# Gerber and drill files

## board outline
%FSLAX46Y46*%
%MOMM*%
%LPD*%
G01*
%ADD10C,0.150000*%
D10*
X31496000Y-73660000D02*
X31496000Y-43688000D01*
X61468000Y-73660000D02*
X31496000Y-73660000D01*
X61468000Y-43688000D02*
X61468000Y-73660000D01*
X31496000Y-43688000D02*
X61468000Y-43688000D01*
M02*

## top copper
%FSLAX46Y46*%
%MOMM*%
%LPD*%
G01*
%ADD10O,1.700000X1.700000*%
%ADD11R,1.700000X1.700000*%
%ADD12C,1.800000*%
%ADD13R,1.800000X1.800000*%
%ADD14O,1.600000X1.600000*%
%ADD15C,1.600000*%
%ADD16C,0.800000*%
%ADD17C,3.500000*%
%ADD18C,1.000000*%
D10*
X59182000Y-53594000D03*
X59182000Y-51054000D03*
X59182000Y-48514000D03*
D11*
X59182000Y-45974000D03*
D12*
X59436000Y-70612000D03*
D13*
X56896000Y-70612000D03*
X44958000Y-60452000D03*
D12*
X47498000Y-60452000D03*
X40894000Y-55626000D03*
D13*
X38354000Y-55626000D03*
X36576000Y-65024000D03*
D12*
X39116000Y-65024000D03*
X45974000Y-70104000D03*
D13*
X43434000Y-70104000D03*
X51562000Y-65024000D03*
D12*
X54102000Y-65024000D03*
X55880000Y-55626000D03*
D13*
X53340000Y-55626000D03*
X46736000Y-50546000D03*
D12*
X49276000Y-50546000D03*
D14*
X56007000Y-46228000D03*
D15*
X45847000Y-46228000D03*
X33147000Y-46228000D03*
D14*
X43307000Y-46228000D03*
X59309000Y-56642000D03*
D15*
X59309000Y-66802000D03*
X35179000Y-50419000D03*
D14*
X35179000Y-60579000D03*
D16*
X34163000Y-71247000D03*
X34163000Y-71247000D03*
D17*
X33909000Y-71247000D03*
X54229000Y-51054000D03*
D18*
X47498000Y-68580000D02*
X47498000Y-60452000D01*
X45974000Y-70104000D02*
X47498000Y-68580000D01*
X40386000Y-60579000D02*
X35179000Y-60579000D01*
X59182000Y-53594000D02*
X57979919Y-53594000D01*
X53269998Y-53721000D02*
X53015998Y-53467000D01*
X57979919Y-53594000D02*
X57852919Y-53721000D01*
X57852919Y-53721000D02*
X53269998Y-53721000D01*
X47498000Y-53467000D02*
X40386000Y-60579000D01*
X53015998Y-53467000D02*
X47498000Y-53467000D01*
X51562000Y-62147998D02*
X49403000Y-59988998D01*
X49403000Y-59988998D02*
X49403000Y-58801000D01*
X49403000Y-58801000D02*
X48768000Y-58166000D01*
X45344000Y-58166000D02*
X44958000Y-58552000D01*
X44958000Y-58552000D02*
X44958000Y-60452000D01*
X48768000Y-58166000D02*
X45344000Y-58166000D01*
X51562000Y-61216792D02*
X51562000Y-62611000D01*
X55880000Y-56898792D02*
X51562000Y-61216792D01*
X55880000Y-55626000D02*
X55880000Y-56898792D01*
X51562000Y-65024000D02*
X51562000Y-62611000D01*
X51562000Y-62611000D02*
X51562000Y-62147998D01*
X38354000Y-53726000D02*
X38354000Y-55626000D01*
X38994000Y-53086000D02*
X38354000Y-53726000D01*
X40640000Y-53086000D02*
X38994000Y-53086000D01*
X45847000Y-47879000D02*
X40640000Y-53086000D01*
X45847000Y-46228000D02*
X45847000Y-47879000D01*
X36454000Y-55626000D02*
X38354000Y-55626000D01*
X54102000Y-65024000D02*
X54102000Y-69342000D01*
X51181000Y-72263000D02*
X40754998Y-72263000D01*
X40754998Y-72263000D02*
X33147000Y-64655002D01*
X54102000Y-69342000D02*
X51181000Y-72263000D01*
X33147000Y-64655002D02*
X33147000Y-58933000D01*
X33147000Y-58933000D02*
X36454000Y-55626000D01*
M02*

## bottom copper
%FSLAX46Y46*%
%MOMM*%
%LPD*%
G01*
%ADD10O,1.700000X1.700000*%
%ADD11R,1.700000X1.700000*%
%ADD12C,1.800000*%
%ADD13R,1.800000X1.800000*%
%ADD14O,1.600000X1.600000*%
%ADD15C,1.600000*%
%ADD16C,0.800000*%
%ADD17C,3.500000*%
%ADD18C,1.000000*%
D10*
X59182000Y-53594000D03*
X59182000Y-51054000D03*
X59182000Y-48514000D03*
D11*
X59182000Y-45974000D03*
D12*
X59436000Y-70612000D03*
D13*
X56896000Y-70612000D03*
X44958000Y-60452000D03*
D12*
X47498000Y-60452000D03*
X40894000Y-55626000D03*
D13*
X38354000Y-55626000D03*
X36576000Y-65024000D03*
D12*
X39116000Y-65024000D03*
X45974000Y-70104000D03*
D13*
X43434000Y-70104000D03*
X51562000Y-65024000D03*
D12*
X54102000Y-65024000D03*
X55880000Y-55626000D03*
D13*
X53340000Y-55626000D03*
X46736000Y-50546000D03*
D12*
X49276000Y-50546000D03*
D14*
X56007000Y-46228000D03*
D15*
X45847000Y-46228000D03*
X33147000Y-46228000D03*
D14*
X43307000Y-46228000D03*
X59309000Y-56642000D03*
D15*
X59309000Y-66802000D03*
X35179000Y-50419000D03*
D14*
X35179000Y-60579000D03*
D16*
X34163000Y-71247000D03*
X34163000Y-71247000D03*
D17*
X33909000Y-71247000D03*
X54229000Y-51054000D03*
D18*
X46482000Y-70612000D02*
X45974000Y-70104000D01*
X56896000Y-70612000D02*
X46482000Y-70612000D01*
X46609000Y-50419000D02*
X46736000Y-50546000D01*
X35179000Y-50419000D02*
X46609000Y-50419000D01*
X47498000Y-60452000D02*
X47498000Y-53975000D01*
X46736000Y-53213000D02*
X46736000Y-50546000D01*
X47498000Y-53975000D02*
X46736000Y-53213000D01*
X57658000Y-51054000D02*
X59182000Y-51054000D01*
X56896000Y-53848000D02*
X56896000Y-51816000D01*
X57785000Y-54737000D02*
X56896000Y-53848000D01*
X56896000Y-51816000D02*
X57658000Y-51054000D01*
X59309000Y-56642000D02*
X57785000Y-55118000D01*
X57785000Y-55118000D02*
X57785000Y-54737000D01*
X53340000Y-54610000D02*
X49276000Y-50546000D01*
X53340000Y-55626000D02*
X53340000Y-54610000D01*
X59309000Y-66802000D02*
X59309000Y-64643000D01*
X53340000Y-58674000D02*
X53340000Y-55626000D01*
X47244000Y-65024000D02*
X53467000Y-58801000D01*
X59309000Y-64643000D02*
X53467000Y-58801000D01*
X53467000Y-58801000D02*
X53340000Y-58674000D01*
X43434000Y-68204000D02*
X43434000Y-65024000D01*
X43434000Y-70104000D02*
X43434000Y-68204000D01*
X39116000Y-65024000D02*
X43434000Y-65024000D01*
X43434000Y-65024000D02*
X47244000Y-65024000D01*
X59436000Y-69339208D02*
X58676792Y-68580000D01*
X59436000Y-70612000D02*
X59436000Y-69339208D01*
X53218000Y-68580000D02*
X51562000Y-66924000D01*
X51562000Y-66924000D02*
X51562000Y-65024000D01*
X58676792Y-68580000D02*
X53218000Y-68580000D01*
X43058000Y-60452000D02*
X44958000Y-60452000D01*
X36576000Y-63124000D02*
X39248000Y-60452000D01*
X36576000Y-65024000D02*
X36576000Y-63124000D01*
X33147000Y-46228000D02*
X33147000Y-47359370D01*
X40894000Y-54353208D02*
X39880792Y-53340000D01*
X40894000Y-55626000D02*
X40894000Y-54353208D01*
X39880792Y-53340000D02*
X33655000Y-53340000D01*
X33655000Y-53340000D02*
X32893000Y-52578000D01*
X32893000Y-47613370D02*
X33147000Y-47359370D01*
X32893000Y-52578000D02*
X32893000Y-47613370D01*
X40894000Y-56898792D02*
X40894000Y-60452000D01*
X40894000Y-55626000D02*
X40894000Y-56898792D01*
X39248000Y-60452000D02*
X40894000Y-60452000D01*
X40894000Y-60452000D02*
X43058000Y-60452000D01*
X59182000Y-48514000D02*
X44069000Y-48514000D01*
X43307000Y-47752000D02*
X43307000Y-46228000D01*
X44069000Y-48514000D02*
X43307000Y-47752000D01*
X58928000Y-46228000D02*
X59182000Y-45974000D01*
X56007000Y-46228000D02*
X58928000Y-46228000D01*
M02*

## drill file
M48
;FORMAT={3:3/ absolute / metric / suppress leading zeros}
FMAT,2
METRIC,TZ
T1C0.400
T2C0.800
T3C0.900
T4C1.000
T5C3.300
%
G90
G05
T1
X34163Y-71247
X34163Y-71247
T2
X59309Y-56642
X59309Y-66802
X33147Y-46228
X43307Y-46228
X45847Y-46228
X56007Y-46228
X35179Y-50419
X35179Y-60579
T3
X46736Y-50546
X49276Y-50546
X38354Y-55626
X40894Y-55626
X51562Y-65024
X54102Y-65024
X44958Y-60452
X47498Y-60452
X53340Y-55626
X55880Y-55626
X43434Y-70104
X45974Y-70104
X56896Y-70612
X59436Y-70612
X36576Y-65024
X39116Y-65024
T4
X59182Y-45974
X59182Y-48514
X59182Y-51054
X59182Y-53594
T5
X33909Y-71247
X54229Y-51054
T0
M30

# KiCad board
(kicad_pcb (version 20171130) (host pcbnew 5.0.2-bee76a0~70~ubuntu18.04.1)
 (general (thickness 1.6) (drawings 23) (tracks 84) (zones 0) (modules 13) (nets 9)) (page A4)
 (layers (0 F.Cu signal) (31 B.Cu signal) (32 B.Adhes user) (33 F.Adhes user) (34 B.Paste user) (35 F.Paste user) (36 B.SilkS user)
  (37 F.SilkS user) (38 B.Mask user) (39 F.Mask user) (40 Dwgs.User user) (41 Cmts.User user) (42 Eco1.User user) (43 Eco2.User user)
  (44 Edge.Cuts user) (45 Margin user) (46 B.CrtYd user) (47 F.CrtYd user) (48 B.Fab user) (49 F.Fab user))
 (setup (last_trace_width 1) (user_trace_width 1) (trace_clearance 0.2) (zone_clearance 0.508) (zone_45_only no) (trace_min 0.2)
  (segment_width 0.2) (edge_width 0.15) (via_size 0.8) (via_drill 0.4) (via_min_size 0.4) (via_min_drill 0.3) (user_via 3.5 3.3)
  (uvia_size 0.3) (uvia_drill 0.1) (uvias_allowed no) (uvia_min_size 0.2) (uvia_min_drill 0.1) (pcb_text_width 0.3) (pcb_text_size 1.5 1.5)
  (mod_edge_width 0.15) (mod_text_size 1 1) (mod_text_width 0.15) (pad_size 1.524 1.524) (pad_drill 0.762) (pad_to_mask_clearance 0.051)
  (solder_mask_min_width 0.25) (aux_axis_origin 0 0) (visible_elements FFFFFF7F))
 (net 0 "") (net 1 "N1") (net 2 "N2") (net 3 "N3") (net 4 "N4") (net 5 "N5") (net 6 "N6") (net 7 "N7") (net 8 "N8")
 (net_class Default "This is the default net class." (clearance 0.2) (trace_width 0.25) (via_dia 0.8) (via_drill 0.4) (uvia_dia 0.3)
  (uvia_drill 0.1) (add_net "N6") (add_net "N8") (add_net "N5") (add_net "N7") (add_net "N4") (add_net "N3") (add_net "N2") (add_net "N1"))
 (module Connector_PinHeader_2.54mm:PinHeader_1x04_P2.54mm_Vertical (layer F.Cu) (at 59.182 45.974)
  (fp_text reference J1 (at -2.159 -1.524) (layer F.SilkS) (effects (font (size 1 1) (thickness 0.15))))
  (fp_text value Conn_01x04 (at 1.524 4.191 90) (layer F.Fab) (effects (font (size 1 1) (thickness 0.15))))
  (pad 4 thru_hole oval (at 0 7.62) (size 1.7 1.7) (drill 1) (layers *.Cu *.Mask) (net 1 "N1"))
  (pad 3 thru_hole oval (at 0 5.08) (size 1.7 1.7) (drill 1) (layers *.Cu *.Mask) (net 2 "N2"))
  (pad 2 thru_hole oval (at 0 2.54) (size 1.7 1.7) (drill 1) (layers *.Cu *.Mask) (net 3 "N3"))
  (pad 1 thru_hole rect (at 0 0) (size 1.7 1.7) (drill 1) (layers *.Cu *.Mask) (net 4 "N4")))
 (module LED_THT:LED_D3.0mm (layer F.Cu) (at 56.896 70.612)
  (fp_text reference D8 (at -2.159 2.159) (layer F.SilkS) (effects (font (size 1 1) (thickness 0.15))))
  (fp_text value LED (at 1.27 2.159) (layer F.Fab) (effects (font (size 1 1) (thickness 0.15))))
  (pad 2 thru_hole circle (at 2.54 0) (size 1.8 1.8) (drill 0.9) (layers *.Cu *.Mask) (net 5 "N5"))
  (pad 1 thru_hole rect (at 0 0) (size 1.8 1.8) (drill 0.9) (layers *.Cu *.Mask) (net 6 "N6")))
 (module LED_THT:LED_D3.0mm (layer F.Cu) (at 44.958 60.452)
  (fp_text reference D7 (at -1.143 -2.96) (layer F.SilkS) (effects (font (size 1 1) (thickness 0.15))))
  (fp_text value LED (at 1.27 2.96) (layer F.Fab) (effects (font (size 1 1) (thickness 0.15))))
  (pad 1 thru_hole rect (at 0 0) (size 1.8 1.8) (drill 0.9) (layers *.Cu *.Mask) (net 5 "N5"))
  (pad 2 thru_hole circle (at 2.54 0) (size 1.8 1.8) (drill 0.9) (layers *.Cu *.Mask) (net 6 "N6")))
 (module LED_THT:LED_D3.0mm (layer F.Cu) (at 38.354 55.626)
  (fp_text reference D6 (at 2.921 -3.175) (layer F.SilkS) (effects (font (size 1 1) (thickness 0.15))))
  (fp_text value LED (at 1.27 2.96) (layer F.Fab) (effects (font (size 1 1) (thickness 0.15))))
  (pad 2 thru_hole circle (at 2.54 0) (size 1.8 1.8) (drill 0.9) (layers *.Cu *.Mask) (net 5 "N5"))
  (pad 1 thru_hole rect (at 0 0) (size 1.8 1.8) (drill 0.9) (layers *.Cu *.Mask) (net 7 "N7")))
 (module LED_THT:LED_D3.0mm (layer F.Cu) (at 36.576 65.024)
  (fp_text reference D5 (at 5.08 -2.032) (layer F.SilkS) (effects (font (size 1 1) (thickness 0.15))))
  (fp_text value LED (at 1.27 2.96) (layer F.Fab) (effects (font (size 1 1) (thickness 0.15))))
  (pad 1 thru_hole rect (at 0 0) (size 1.8 1.8) (drill 0.9) (layers *.Cu *.Mask) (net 5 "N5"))
  (pad 2 thru_hole circle (at 2.54 0) (size 1.8 1.8) (drill 0.9) (layers *.Cu *.Mask) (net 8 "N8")))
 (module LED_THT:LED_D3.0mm (layer F.Cu) (at 43.434 70.104)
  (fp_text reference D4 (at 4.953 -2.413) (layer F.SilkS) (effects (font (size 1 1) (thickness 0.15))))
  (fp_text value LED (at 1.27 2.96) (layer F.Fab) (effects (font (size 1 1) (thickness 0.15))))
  (pad 2 thru_hole circle (at 2.54 0) (size 1.8 1.8) (drill 0.9) (layers *.Cu *.Mask) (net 6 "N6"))
  (pad 1 thru_hole rect (at 0 0) (size 1.8 1.8) (drill 0.9) (layers *.Cu *.Mask) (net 8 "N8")))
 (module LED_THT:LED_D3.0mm (layer F.Cu) (at 51.562 65.024)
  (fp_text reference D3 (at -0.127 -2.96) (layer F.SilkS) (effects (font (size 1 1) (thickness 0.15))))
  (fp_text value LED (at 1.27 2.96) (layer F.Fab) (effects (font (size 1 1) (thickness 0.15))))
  (pad 1 thru_hole rect (at 0 0) (size 1.8 1.8) (drill 0.9) (layers *.Cu *.Mask) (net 5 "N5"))
  (pad 2 thru_hole circle (at 2.54 0) (size 1.8 1.8) (drill 0.9) (layers *.Cu *.Mask) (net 7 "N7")))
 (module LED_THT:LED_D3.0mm (layer F.Cu) (at 53.34 55.626)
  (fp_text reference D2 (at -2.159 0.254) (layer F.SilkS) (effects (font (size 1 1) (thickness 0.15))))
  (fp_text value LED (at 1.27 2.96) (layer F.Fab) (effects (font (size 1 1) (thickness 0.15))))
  (pad 2 thru_hole circle (at 2.54 0) (size 1.8 1.8) (drill 0.9) (layers *.Cu *.Mask) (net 5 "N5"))
  (pad 1 thru_hole rect (at 0 0) (size 1.8 1.8) (drill 0.9) (layers *.Cu *.Mask) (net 8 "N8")))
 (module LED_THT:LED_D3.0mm (layer F.Cu) (at 46.736 50.546)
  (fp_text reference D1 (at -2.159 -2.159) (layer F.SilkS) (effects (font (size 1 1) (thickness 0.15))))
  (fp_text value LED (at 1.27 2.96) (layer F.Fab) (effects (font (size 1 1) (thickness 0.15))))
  (pad 1 thru_hole rect (at 0 0) (size 1.8 1.8) (drill 0.9) (layers *.Cu *.Mask) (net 6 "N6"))
  (pad 2 thru_hole circle (at 2.54 0) (size 1.8 1.8) (drill 0.9) (layers *.Cu *.Mask) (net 8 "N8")))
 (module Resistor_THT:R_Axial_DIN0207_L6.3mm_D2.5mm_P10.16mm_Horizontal (layer F.Cu) (at 45.847 46.228)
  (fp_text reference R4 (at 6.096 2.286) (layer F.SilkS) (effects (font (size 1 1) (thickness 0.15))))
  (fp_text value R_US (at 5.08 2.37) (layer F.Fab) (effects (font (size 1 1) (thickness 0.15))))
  (pad 2 thru_hole oval (at 10.16 0) (size 1.6 1.6) (drill 0.8) (layers *.Cu *.Mask) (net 4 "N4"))
  (pad 1 thru_hole circle (at 0 0) (size 1.6 1.6) (drill 0.8) (layers *.Cu *.Mask) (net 7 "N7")))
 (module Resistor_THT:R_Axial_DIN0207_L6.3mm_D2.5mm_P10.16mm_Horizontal (layer F.Cu) (at 33.147 46.228)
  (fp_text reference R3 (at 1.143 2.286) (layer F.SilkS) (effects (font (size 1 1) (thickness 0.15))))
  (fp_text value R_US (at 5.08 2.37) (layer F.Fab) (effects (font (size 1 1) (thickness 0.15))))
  (pad 1 thru_hole circle (at 0 0) (size 1.6 1.6) (drill 0.8) (layers *.Cu *.Mask) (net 5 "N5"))
  (pad 2 thru_hole oval (at 10.16 0) (size 1.6 1.6) (drill 0.8) (layers *.Cu *.Mask) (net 3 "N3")))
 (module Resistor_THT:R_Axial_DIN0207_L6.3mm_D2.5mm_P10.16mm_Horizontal (layer F.Cu) (at 59.309 66.802 90)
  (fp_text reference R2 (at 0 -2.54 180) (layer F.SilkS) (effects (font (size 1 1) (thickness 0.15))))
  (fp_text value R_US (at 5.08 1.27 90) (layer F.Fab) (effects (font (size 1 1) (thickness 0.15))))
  (pad 2 thru_hole oval (at 10.16 0 90) (size 1.6 1.6) (drill 0.8) (layers *.Cu *.Mask) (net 2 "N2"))
  (pad 1 thru_hole circle (at 0 0 90) (size 1.6 1.6) (drill 0.8) (layers *.Cu *.Mask) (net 8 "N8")))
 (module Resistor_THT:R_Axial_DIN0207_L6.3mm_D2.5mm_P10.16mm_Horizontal (layer F.Cu) (at 35.179 50.419 270)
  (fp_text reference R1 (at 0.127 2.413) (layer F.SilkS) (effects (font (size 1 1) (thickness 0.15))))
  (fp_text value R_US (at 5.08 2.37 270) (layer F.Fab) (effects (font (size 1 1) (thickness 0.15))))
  (pad 1 thru_hole circle (at 0 0 270) (size 1.6 1.6) (drill 0.8) (layers *.Cu *.Mask) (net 6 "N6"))
  (pad 2 thru_hole oval (at 10.16 0 270) (size 1.6 1.6) (drill 0.8) (layers *.Cu *.Mask) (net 1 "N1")))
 (gr_line (start 31.496 73.66) (end 31.496 43.688) (layer Edge.Cuts) (width 0.15))
 (gr_line (start 61.468 73.66) (end 31.496 73.66) (layer Edge.Cuts) (width 0.15))
 (gr_line (start 61.468 43.688) (end 61.468 73.66) (layer Edge.Cuts) (width 0.15))
 (gr_line (start 31.496 43.688) (end 61.468 43.688) (layer Edge.Cuts) (width 0.15))
 (via (at 34.163 71.247) (size 0.8) (drill 0.4) (layers F.Cu B.Cu) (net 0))
 (via (at 34.163 71.247) (size 0.8) (drill 0.4) (layers F.Cu B.Cu) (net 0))
 (via (at 33.909 71.247) (size 3.5) (drill 3.3) (layers F.Cu B.Cu) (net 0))
 (via (at 54.229 51.054) (size 3.5) (drill 3.3) (layers F.Cu B.Cu) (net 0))
 (segment (start 46.482 70.612) (end 45.974 70.104) (width 1) (layer B.Cu) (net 6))
 (segment (start 56.896 70.612) (end 46.482 70.612) (width 1) (layer B.Cu) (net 6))
 (segment (start 46.609 50.419) (end 46.736 50.546) (width 1) (layer B.Cu) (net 6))
 (segment (start 35.179 50.419) (end 46.609 50.419) (width 1) (layer B.Cu) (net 6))
 (segment (start 47.498 68.58) (end 47.498 60.452) (width 1) (layer F.Cu) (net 6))
 (segment (start 45.974 70.104) (end 47.498 68.58) (width 1) (layer F.Cu) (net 6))
 (segment (start 47.498 60.452) (end 47.498 53.975) (width 1) (layer B.Cu) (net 6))
 (segment (start 46.736 53.213) (end 46.736 50.546) (width 1) (layer B.Cu) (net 6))
 (segment (start 47.498 53.975) (end 46.736 53.213) (width 1) (layer B.Cu) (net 6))
 (segment (start 40.386 60.579) (end 35.179 60.579) (width 1) (layer F.Cu) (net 1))
 (segment (start 59.182 53.594) (end 57.979919 53.594) (width 1) (layer F.Cu) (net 1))
 (segment (start 53.269998 53.721) (end 53.015998 53.467) (width 1) (layer F.Cu) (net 1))
 (segment (start 57.979919 53.594) (end 57.852919 53.721) (width 1) (layer F.Cu) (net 1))
 (segment (start 57.852919 53.721) (end 53.269998 53.721) (width 1) (layer F.Cu) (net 1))
 (segment (start 47.498 53.467) (end 40.386 60.579) (width 1) (layer F.Cu) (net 1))
 (segment (start 53.015998 53.467) (end 47.498 53.467) (width 1) (layer F.Cu) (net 1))
 (segment (start 57.658 51.054) (end 59.182 51.054) (width 1) (layer B.Cu) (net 2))
 (segment (start 56.896 53.848) (end 56.896 51.816) (width 1) (layer B.Cu) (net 2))
 (segment (start 57.785 54.737) (end 56.896 53.848) (width 1) (layer B.Cu) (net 2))
 (segment (start 56.896 51.816) (end 57.658 51.054) (width 1) (layer B.Cu) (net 2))
 (segment (start 59.309 56.642) (end 57.785 55.118) (width 1) (layer B.Cu) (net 2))
 (segment (start 57.785 55.118) (end 57.785 54.737) (width 1) (layer B.Cu) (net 2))
 (segment (start 53.34 54.61) (end 49.276 50.546) (width 1) (layer B.Cu) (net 8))
 (segment (start 53.34 55.626) (end 53.34 54.61) (width 1) (layer B.Cu) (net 8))
 (segment (start 59.309 66.802) (end 59.309 64.643) (width 1) (layer B.Cu) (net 8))
 (segment (start 53.34 58.674) (end 53.34 55.626) (width 1) (layer B.Cu) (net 8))
 (segment (start 47.244 65.024) (end 53.467 58.801) (width 1) (layer B.Cu) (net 8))
 (segment (start 59.309 64.643) (end 53.467 58.801) (width 1) (layer B.Cu) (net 8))
 (segment (start 53.467 58.801) (end 53.34 58.674) (width 1) (layer B.Cu) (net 8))
 (segment (start 43.434 68.204) (end 43.434 65.024) (width 1) (layer B.Cu) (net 8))
 (segment (start 43.434 70.104) (end 43.434 68.204) (width 1) (layer B.Cu) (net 8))
 (segment (start 39.116 65.024) (end 43.434 65.024) (width 1) (layer B.Cu) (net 8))
 (segment (start 43.434 65.024) (end 47.244 65.024) (width 1) (layer B.Cu) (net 8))
 (segment (start 59.436 69.339208) (end 58.676792 68.58) (width 1) (layer B.Cu) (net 5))
 (segment (start 59.436 70.612) (end 59.436 69.339208) (width 1) (layer B.Cu) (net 5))
 (segment (start 53.218 68.58) (end 51.562 66.924) (width 1) (layer B.Cu) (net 5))
 (segment (start 51.562 66.924) (end 51.562 65.024) (width 1) (layer B.Cu) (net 5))
 (segment (start 58.676792 68.58) (end 53.218 68.58) (width 1) (layer B.Cu) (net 5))
 (segment (start 43.058 60.452) (end 44.958 60.452) (width 1) (layer B.Cu) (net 5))
 (segment (start 36.576 63.124) (end 39.248 60.452) (width 1) (layer B.Cu) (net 5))
 (segment (start 36.576 65.024) (end 36.576 63.124) (width 1) (layer B.Cu) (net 5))
 (segment (start 33.147 46.228) (end 33.147 47.35937) (width 1) (layer B.Cu) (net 5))
 (segment (start 40.894 54.353208) (end 39.880792 53.34) (width 1) (layer B.Cu) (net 5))
 (segment (start 40.894 55.626) (end 40.894 54.353208) (width 1) (layer B.Cu) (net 5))
 (segment (start 39.880792 53.34) (end 33.655 53.34) (width 1) (layer B.Cu) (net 5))
 (segment (start 33.655 53.34) (end 32.893 52.578) (width 1) (layer B.Cu) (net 5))
 (segment (start 32.893 47.61337) (end 33.147 47.35937) (width 1) (layer B.Cu) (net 5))
 (segment (start 32.893 52.578) (end 32.893 47.61337) (width 1) (layer B.Cu) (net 5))
 (segment (start 40.894 56.898792) (end 40.894 60.452) (width 1) (layer B.Cu) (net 5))
 (segment (start 40.894 55.626) (end 40.894 56.898792) (width 1) (layer B.Cu) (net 5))
 (segment (start 39.248 60.452) (end 40.894 60.452) (width 1) (layer B.Cu) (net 5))
 (segment (start 40.894 60.452) (end 43.058 60.452) (width 1) (layer B.Cu) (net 5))
 (segment (start 51.562 62.147998) (end 49.403 59.988998) (width 1) (layer F.Cu) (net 5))
 (segment (start 49.403 59.988998) (end 49.403 58.801) (width 1) (layer F.Cu) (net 5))
 (segment (start 49.403 58.801) (end 48.768 58.166) (width 1) (layer F.Cu) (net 5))
 (segment (start 45.344 58.166) (end 44.958 58.552) (width 1) (layer F.Cu) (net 5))
 (segment (start 44.958 58.552) (end 44.958 60.452) (width 1) (layer F.Cu) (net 5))
 (segment (start 48.768 58.166) (end 45.344 58.166) (width 1) (layer F.Cu) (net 5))
 (segment (start 51.562 61.216792) (end 51.562 62.611) (width 1) (layer F.Cu) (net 5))
 (segment (start 55.88 56.898792) (end 51.562 61.216792) (width 1) (layer F.Cu) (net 5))
 (segment (start 55.88 55.626) (end 55.88 56.898792) (width 1) (layer F.Cu) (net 5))
 (segment (start 51.562 65.024) (end 51.562 62.611) (width 1) (layer F.Cu) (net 5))
 (segment (start 51.562 62.611) (end 51.562 62.147998) (width 1) (layer F.Cu) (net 5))
 (segment (start 59.182 48.514) (end 44.069 48.514) (width 1) (layer B.Cu) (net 3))
 (segment (start 43.307 47.752) (end 43.307 46.228) (width 1) (layer B.Cu) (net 3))
 (segment (start 44.069 48.514) (end 43.307 47.752) (width 1) (layer B.Cu) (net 3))
 (segment (start 58.928 46.228) (end 59.182 45.974) (width 1) (layer B.Cu) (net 4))
 (segment (start 56.007 46.228) (end 58.928 46.228) (width 1) (layer B.Cu) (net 4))
 (segment (start 38.354 53.726) (end 38.354 55.626) (width 1) (layer F.Cu) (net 7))
 (segment (start 38.994 53.086) (end 38.354 53.726) (width 1) (layer F.Cu) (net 7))
 (segment (start 40.64 53.086) (end 38.994 53.086) (width 1) (layer F.Cu) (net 7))
 (segment (start 45.847 47.879) (end 40.64 53.086) (width 1) (layer F.Cu) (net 7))
 (segment (start 45.847 46.228) (end 45.847 47.879) (width 1) (layer F.Cu) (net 7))
 (segment (start 36.454 55.626) (end 38.354 55.626) (width 1) (layer F.Cu) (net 7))
 (segment (start 54.102 65.024) (end 54.102 69.342) (width 1) (layer F.Cu) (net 7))
 (segment (start 51.181 72.263) (end 40.754998 72.263) (width 1) (layer F.Cu) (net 7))
 (segment (start 40.754998 72.263) (end 33.147 64.655002) (width 1) (layer F.Cu) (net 7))
 (segment (start 54.102 69.342) (end 51.181 72.263) (width 1) (layer F.Cu) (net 7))
 (segment (start 33.147 64.655002) (end 33.147 58.933) (width 1) (layer F.Cu) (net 7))
 (segment (start 33.147 58.933) (end 36.454 55.626) (width 1) (layer F.Cu) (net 7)))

